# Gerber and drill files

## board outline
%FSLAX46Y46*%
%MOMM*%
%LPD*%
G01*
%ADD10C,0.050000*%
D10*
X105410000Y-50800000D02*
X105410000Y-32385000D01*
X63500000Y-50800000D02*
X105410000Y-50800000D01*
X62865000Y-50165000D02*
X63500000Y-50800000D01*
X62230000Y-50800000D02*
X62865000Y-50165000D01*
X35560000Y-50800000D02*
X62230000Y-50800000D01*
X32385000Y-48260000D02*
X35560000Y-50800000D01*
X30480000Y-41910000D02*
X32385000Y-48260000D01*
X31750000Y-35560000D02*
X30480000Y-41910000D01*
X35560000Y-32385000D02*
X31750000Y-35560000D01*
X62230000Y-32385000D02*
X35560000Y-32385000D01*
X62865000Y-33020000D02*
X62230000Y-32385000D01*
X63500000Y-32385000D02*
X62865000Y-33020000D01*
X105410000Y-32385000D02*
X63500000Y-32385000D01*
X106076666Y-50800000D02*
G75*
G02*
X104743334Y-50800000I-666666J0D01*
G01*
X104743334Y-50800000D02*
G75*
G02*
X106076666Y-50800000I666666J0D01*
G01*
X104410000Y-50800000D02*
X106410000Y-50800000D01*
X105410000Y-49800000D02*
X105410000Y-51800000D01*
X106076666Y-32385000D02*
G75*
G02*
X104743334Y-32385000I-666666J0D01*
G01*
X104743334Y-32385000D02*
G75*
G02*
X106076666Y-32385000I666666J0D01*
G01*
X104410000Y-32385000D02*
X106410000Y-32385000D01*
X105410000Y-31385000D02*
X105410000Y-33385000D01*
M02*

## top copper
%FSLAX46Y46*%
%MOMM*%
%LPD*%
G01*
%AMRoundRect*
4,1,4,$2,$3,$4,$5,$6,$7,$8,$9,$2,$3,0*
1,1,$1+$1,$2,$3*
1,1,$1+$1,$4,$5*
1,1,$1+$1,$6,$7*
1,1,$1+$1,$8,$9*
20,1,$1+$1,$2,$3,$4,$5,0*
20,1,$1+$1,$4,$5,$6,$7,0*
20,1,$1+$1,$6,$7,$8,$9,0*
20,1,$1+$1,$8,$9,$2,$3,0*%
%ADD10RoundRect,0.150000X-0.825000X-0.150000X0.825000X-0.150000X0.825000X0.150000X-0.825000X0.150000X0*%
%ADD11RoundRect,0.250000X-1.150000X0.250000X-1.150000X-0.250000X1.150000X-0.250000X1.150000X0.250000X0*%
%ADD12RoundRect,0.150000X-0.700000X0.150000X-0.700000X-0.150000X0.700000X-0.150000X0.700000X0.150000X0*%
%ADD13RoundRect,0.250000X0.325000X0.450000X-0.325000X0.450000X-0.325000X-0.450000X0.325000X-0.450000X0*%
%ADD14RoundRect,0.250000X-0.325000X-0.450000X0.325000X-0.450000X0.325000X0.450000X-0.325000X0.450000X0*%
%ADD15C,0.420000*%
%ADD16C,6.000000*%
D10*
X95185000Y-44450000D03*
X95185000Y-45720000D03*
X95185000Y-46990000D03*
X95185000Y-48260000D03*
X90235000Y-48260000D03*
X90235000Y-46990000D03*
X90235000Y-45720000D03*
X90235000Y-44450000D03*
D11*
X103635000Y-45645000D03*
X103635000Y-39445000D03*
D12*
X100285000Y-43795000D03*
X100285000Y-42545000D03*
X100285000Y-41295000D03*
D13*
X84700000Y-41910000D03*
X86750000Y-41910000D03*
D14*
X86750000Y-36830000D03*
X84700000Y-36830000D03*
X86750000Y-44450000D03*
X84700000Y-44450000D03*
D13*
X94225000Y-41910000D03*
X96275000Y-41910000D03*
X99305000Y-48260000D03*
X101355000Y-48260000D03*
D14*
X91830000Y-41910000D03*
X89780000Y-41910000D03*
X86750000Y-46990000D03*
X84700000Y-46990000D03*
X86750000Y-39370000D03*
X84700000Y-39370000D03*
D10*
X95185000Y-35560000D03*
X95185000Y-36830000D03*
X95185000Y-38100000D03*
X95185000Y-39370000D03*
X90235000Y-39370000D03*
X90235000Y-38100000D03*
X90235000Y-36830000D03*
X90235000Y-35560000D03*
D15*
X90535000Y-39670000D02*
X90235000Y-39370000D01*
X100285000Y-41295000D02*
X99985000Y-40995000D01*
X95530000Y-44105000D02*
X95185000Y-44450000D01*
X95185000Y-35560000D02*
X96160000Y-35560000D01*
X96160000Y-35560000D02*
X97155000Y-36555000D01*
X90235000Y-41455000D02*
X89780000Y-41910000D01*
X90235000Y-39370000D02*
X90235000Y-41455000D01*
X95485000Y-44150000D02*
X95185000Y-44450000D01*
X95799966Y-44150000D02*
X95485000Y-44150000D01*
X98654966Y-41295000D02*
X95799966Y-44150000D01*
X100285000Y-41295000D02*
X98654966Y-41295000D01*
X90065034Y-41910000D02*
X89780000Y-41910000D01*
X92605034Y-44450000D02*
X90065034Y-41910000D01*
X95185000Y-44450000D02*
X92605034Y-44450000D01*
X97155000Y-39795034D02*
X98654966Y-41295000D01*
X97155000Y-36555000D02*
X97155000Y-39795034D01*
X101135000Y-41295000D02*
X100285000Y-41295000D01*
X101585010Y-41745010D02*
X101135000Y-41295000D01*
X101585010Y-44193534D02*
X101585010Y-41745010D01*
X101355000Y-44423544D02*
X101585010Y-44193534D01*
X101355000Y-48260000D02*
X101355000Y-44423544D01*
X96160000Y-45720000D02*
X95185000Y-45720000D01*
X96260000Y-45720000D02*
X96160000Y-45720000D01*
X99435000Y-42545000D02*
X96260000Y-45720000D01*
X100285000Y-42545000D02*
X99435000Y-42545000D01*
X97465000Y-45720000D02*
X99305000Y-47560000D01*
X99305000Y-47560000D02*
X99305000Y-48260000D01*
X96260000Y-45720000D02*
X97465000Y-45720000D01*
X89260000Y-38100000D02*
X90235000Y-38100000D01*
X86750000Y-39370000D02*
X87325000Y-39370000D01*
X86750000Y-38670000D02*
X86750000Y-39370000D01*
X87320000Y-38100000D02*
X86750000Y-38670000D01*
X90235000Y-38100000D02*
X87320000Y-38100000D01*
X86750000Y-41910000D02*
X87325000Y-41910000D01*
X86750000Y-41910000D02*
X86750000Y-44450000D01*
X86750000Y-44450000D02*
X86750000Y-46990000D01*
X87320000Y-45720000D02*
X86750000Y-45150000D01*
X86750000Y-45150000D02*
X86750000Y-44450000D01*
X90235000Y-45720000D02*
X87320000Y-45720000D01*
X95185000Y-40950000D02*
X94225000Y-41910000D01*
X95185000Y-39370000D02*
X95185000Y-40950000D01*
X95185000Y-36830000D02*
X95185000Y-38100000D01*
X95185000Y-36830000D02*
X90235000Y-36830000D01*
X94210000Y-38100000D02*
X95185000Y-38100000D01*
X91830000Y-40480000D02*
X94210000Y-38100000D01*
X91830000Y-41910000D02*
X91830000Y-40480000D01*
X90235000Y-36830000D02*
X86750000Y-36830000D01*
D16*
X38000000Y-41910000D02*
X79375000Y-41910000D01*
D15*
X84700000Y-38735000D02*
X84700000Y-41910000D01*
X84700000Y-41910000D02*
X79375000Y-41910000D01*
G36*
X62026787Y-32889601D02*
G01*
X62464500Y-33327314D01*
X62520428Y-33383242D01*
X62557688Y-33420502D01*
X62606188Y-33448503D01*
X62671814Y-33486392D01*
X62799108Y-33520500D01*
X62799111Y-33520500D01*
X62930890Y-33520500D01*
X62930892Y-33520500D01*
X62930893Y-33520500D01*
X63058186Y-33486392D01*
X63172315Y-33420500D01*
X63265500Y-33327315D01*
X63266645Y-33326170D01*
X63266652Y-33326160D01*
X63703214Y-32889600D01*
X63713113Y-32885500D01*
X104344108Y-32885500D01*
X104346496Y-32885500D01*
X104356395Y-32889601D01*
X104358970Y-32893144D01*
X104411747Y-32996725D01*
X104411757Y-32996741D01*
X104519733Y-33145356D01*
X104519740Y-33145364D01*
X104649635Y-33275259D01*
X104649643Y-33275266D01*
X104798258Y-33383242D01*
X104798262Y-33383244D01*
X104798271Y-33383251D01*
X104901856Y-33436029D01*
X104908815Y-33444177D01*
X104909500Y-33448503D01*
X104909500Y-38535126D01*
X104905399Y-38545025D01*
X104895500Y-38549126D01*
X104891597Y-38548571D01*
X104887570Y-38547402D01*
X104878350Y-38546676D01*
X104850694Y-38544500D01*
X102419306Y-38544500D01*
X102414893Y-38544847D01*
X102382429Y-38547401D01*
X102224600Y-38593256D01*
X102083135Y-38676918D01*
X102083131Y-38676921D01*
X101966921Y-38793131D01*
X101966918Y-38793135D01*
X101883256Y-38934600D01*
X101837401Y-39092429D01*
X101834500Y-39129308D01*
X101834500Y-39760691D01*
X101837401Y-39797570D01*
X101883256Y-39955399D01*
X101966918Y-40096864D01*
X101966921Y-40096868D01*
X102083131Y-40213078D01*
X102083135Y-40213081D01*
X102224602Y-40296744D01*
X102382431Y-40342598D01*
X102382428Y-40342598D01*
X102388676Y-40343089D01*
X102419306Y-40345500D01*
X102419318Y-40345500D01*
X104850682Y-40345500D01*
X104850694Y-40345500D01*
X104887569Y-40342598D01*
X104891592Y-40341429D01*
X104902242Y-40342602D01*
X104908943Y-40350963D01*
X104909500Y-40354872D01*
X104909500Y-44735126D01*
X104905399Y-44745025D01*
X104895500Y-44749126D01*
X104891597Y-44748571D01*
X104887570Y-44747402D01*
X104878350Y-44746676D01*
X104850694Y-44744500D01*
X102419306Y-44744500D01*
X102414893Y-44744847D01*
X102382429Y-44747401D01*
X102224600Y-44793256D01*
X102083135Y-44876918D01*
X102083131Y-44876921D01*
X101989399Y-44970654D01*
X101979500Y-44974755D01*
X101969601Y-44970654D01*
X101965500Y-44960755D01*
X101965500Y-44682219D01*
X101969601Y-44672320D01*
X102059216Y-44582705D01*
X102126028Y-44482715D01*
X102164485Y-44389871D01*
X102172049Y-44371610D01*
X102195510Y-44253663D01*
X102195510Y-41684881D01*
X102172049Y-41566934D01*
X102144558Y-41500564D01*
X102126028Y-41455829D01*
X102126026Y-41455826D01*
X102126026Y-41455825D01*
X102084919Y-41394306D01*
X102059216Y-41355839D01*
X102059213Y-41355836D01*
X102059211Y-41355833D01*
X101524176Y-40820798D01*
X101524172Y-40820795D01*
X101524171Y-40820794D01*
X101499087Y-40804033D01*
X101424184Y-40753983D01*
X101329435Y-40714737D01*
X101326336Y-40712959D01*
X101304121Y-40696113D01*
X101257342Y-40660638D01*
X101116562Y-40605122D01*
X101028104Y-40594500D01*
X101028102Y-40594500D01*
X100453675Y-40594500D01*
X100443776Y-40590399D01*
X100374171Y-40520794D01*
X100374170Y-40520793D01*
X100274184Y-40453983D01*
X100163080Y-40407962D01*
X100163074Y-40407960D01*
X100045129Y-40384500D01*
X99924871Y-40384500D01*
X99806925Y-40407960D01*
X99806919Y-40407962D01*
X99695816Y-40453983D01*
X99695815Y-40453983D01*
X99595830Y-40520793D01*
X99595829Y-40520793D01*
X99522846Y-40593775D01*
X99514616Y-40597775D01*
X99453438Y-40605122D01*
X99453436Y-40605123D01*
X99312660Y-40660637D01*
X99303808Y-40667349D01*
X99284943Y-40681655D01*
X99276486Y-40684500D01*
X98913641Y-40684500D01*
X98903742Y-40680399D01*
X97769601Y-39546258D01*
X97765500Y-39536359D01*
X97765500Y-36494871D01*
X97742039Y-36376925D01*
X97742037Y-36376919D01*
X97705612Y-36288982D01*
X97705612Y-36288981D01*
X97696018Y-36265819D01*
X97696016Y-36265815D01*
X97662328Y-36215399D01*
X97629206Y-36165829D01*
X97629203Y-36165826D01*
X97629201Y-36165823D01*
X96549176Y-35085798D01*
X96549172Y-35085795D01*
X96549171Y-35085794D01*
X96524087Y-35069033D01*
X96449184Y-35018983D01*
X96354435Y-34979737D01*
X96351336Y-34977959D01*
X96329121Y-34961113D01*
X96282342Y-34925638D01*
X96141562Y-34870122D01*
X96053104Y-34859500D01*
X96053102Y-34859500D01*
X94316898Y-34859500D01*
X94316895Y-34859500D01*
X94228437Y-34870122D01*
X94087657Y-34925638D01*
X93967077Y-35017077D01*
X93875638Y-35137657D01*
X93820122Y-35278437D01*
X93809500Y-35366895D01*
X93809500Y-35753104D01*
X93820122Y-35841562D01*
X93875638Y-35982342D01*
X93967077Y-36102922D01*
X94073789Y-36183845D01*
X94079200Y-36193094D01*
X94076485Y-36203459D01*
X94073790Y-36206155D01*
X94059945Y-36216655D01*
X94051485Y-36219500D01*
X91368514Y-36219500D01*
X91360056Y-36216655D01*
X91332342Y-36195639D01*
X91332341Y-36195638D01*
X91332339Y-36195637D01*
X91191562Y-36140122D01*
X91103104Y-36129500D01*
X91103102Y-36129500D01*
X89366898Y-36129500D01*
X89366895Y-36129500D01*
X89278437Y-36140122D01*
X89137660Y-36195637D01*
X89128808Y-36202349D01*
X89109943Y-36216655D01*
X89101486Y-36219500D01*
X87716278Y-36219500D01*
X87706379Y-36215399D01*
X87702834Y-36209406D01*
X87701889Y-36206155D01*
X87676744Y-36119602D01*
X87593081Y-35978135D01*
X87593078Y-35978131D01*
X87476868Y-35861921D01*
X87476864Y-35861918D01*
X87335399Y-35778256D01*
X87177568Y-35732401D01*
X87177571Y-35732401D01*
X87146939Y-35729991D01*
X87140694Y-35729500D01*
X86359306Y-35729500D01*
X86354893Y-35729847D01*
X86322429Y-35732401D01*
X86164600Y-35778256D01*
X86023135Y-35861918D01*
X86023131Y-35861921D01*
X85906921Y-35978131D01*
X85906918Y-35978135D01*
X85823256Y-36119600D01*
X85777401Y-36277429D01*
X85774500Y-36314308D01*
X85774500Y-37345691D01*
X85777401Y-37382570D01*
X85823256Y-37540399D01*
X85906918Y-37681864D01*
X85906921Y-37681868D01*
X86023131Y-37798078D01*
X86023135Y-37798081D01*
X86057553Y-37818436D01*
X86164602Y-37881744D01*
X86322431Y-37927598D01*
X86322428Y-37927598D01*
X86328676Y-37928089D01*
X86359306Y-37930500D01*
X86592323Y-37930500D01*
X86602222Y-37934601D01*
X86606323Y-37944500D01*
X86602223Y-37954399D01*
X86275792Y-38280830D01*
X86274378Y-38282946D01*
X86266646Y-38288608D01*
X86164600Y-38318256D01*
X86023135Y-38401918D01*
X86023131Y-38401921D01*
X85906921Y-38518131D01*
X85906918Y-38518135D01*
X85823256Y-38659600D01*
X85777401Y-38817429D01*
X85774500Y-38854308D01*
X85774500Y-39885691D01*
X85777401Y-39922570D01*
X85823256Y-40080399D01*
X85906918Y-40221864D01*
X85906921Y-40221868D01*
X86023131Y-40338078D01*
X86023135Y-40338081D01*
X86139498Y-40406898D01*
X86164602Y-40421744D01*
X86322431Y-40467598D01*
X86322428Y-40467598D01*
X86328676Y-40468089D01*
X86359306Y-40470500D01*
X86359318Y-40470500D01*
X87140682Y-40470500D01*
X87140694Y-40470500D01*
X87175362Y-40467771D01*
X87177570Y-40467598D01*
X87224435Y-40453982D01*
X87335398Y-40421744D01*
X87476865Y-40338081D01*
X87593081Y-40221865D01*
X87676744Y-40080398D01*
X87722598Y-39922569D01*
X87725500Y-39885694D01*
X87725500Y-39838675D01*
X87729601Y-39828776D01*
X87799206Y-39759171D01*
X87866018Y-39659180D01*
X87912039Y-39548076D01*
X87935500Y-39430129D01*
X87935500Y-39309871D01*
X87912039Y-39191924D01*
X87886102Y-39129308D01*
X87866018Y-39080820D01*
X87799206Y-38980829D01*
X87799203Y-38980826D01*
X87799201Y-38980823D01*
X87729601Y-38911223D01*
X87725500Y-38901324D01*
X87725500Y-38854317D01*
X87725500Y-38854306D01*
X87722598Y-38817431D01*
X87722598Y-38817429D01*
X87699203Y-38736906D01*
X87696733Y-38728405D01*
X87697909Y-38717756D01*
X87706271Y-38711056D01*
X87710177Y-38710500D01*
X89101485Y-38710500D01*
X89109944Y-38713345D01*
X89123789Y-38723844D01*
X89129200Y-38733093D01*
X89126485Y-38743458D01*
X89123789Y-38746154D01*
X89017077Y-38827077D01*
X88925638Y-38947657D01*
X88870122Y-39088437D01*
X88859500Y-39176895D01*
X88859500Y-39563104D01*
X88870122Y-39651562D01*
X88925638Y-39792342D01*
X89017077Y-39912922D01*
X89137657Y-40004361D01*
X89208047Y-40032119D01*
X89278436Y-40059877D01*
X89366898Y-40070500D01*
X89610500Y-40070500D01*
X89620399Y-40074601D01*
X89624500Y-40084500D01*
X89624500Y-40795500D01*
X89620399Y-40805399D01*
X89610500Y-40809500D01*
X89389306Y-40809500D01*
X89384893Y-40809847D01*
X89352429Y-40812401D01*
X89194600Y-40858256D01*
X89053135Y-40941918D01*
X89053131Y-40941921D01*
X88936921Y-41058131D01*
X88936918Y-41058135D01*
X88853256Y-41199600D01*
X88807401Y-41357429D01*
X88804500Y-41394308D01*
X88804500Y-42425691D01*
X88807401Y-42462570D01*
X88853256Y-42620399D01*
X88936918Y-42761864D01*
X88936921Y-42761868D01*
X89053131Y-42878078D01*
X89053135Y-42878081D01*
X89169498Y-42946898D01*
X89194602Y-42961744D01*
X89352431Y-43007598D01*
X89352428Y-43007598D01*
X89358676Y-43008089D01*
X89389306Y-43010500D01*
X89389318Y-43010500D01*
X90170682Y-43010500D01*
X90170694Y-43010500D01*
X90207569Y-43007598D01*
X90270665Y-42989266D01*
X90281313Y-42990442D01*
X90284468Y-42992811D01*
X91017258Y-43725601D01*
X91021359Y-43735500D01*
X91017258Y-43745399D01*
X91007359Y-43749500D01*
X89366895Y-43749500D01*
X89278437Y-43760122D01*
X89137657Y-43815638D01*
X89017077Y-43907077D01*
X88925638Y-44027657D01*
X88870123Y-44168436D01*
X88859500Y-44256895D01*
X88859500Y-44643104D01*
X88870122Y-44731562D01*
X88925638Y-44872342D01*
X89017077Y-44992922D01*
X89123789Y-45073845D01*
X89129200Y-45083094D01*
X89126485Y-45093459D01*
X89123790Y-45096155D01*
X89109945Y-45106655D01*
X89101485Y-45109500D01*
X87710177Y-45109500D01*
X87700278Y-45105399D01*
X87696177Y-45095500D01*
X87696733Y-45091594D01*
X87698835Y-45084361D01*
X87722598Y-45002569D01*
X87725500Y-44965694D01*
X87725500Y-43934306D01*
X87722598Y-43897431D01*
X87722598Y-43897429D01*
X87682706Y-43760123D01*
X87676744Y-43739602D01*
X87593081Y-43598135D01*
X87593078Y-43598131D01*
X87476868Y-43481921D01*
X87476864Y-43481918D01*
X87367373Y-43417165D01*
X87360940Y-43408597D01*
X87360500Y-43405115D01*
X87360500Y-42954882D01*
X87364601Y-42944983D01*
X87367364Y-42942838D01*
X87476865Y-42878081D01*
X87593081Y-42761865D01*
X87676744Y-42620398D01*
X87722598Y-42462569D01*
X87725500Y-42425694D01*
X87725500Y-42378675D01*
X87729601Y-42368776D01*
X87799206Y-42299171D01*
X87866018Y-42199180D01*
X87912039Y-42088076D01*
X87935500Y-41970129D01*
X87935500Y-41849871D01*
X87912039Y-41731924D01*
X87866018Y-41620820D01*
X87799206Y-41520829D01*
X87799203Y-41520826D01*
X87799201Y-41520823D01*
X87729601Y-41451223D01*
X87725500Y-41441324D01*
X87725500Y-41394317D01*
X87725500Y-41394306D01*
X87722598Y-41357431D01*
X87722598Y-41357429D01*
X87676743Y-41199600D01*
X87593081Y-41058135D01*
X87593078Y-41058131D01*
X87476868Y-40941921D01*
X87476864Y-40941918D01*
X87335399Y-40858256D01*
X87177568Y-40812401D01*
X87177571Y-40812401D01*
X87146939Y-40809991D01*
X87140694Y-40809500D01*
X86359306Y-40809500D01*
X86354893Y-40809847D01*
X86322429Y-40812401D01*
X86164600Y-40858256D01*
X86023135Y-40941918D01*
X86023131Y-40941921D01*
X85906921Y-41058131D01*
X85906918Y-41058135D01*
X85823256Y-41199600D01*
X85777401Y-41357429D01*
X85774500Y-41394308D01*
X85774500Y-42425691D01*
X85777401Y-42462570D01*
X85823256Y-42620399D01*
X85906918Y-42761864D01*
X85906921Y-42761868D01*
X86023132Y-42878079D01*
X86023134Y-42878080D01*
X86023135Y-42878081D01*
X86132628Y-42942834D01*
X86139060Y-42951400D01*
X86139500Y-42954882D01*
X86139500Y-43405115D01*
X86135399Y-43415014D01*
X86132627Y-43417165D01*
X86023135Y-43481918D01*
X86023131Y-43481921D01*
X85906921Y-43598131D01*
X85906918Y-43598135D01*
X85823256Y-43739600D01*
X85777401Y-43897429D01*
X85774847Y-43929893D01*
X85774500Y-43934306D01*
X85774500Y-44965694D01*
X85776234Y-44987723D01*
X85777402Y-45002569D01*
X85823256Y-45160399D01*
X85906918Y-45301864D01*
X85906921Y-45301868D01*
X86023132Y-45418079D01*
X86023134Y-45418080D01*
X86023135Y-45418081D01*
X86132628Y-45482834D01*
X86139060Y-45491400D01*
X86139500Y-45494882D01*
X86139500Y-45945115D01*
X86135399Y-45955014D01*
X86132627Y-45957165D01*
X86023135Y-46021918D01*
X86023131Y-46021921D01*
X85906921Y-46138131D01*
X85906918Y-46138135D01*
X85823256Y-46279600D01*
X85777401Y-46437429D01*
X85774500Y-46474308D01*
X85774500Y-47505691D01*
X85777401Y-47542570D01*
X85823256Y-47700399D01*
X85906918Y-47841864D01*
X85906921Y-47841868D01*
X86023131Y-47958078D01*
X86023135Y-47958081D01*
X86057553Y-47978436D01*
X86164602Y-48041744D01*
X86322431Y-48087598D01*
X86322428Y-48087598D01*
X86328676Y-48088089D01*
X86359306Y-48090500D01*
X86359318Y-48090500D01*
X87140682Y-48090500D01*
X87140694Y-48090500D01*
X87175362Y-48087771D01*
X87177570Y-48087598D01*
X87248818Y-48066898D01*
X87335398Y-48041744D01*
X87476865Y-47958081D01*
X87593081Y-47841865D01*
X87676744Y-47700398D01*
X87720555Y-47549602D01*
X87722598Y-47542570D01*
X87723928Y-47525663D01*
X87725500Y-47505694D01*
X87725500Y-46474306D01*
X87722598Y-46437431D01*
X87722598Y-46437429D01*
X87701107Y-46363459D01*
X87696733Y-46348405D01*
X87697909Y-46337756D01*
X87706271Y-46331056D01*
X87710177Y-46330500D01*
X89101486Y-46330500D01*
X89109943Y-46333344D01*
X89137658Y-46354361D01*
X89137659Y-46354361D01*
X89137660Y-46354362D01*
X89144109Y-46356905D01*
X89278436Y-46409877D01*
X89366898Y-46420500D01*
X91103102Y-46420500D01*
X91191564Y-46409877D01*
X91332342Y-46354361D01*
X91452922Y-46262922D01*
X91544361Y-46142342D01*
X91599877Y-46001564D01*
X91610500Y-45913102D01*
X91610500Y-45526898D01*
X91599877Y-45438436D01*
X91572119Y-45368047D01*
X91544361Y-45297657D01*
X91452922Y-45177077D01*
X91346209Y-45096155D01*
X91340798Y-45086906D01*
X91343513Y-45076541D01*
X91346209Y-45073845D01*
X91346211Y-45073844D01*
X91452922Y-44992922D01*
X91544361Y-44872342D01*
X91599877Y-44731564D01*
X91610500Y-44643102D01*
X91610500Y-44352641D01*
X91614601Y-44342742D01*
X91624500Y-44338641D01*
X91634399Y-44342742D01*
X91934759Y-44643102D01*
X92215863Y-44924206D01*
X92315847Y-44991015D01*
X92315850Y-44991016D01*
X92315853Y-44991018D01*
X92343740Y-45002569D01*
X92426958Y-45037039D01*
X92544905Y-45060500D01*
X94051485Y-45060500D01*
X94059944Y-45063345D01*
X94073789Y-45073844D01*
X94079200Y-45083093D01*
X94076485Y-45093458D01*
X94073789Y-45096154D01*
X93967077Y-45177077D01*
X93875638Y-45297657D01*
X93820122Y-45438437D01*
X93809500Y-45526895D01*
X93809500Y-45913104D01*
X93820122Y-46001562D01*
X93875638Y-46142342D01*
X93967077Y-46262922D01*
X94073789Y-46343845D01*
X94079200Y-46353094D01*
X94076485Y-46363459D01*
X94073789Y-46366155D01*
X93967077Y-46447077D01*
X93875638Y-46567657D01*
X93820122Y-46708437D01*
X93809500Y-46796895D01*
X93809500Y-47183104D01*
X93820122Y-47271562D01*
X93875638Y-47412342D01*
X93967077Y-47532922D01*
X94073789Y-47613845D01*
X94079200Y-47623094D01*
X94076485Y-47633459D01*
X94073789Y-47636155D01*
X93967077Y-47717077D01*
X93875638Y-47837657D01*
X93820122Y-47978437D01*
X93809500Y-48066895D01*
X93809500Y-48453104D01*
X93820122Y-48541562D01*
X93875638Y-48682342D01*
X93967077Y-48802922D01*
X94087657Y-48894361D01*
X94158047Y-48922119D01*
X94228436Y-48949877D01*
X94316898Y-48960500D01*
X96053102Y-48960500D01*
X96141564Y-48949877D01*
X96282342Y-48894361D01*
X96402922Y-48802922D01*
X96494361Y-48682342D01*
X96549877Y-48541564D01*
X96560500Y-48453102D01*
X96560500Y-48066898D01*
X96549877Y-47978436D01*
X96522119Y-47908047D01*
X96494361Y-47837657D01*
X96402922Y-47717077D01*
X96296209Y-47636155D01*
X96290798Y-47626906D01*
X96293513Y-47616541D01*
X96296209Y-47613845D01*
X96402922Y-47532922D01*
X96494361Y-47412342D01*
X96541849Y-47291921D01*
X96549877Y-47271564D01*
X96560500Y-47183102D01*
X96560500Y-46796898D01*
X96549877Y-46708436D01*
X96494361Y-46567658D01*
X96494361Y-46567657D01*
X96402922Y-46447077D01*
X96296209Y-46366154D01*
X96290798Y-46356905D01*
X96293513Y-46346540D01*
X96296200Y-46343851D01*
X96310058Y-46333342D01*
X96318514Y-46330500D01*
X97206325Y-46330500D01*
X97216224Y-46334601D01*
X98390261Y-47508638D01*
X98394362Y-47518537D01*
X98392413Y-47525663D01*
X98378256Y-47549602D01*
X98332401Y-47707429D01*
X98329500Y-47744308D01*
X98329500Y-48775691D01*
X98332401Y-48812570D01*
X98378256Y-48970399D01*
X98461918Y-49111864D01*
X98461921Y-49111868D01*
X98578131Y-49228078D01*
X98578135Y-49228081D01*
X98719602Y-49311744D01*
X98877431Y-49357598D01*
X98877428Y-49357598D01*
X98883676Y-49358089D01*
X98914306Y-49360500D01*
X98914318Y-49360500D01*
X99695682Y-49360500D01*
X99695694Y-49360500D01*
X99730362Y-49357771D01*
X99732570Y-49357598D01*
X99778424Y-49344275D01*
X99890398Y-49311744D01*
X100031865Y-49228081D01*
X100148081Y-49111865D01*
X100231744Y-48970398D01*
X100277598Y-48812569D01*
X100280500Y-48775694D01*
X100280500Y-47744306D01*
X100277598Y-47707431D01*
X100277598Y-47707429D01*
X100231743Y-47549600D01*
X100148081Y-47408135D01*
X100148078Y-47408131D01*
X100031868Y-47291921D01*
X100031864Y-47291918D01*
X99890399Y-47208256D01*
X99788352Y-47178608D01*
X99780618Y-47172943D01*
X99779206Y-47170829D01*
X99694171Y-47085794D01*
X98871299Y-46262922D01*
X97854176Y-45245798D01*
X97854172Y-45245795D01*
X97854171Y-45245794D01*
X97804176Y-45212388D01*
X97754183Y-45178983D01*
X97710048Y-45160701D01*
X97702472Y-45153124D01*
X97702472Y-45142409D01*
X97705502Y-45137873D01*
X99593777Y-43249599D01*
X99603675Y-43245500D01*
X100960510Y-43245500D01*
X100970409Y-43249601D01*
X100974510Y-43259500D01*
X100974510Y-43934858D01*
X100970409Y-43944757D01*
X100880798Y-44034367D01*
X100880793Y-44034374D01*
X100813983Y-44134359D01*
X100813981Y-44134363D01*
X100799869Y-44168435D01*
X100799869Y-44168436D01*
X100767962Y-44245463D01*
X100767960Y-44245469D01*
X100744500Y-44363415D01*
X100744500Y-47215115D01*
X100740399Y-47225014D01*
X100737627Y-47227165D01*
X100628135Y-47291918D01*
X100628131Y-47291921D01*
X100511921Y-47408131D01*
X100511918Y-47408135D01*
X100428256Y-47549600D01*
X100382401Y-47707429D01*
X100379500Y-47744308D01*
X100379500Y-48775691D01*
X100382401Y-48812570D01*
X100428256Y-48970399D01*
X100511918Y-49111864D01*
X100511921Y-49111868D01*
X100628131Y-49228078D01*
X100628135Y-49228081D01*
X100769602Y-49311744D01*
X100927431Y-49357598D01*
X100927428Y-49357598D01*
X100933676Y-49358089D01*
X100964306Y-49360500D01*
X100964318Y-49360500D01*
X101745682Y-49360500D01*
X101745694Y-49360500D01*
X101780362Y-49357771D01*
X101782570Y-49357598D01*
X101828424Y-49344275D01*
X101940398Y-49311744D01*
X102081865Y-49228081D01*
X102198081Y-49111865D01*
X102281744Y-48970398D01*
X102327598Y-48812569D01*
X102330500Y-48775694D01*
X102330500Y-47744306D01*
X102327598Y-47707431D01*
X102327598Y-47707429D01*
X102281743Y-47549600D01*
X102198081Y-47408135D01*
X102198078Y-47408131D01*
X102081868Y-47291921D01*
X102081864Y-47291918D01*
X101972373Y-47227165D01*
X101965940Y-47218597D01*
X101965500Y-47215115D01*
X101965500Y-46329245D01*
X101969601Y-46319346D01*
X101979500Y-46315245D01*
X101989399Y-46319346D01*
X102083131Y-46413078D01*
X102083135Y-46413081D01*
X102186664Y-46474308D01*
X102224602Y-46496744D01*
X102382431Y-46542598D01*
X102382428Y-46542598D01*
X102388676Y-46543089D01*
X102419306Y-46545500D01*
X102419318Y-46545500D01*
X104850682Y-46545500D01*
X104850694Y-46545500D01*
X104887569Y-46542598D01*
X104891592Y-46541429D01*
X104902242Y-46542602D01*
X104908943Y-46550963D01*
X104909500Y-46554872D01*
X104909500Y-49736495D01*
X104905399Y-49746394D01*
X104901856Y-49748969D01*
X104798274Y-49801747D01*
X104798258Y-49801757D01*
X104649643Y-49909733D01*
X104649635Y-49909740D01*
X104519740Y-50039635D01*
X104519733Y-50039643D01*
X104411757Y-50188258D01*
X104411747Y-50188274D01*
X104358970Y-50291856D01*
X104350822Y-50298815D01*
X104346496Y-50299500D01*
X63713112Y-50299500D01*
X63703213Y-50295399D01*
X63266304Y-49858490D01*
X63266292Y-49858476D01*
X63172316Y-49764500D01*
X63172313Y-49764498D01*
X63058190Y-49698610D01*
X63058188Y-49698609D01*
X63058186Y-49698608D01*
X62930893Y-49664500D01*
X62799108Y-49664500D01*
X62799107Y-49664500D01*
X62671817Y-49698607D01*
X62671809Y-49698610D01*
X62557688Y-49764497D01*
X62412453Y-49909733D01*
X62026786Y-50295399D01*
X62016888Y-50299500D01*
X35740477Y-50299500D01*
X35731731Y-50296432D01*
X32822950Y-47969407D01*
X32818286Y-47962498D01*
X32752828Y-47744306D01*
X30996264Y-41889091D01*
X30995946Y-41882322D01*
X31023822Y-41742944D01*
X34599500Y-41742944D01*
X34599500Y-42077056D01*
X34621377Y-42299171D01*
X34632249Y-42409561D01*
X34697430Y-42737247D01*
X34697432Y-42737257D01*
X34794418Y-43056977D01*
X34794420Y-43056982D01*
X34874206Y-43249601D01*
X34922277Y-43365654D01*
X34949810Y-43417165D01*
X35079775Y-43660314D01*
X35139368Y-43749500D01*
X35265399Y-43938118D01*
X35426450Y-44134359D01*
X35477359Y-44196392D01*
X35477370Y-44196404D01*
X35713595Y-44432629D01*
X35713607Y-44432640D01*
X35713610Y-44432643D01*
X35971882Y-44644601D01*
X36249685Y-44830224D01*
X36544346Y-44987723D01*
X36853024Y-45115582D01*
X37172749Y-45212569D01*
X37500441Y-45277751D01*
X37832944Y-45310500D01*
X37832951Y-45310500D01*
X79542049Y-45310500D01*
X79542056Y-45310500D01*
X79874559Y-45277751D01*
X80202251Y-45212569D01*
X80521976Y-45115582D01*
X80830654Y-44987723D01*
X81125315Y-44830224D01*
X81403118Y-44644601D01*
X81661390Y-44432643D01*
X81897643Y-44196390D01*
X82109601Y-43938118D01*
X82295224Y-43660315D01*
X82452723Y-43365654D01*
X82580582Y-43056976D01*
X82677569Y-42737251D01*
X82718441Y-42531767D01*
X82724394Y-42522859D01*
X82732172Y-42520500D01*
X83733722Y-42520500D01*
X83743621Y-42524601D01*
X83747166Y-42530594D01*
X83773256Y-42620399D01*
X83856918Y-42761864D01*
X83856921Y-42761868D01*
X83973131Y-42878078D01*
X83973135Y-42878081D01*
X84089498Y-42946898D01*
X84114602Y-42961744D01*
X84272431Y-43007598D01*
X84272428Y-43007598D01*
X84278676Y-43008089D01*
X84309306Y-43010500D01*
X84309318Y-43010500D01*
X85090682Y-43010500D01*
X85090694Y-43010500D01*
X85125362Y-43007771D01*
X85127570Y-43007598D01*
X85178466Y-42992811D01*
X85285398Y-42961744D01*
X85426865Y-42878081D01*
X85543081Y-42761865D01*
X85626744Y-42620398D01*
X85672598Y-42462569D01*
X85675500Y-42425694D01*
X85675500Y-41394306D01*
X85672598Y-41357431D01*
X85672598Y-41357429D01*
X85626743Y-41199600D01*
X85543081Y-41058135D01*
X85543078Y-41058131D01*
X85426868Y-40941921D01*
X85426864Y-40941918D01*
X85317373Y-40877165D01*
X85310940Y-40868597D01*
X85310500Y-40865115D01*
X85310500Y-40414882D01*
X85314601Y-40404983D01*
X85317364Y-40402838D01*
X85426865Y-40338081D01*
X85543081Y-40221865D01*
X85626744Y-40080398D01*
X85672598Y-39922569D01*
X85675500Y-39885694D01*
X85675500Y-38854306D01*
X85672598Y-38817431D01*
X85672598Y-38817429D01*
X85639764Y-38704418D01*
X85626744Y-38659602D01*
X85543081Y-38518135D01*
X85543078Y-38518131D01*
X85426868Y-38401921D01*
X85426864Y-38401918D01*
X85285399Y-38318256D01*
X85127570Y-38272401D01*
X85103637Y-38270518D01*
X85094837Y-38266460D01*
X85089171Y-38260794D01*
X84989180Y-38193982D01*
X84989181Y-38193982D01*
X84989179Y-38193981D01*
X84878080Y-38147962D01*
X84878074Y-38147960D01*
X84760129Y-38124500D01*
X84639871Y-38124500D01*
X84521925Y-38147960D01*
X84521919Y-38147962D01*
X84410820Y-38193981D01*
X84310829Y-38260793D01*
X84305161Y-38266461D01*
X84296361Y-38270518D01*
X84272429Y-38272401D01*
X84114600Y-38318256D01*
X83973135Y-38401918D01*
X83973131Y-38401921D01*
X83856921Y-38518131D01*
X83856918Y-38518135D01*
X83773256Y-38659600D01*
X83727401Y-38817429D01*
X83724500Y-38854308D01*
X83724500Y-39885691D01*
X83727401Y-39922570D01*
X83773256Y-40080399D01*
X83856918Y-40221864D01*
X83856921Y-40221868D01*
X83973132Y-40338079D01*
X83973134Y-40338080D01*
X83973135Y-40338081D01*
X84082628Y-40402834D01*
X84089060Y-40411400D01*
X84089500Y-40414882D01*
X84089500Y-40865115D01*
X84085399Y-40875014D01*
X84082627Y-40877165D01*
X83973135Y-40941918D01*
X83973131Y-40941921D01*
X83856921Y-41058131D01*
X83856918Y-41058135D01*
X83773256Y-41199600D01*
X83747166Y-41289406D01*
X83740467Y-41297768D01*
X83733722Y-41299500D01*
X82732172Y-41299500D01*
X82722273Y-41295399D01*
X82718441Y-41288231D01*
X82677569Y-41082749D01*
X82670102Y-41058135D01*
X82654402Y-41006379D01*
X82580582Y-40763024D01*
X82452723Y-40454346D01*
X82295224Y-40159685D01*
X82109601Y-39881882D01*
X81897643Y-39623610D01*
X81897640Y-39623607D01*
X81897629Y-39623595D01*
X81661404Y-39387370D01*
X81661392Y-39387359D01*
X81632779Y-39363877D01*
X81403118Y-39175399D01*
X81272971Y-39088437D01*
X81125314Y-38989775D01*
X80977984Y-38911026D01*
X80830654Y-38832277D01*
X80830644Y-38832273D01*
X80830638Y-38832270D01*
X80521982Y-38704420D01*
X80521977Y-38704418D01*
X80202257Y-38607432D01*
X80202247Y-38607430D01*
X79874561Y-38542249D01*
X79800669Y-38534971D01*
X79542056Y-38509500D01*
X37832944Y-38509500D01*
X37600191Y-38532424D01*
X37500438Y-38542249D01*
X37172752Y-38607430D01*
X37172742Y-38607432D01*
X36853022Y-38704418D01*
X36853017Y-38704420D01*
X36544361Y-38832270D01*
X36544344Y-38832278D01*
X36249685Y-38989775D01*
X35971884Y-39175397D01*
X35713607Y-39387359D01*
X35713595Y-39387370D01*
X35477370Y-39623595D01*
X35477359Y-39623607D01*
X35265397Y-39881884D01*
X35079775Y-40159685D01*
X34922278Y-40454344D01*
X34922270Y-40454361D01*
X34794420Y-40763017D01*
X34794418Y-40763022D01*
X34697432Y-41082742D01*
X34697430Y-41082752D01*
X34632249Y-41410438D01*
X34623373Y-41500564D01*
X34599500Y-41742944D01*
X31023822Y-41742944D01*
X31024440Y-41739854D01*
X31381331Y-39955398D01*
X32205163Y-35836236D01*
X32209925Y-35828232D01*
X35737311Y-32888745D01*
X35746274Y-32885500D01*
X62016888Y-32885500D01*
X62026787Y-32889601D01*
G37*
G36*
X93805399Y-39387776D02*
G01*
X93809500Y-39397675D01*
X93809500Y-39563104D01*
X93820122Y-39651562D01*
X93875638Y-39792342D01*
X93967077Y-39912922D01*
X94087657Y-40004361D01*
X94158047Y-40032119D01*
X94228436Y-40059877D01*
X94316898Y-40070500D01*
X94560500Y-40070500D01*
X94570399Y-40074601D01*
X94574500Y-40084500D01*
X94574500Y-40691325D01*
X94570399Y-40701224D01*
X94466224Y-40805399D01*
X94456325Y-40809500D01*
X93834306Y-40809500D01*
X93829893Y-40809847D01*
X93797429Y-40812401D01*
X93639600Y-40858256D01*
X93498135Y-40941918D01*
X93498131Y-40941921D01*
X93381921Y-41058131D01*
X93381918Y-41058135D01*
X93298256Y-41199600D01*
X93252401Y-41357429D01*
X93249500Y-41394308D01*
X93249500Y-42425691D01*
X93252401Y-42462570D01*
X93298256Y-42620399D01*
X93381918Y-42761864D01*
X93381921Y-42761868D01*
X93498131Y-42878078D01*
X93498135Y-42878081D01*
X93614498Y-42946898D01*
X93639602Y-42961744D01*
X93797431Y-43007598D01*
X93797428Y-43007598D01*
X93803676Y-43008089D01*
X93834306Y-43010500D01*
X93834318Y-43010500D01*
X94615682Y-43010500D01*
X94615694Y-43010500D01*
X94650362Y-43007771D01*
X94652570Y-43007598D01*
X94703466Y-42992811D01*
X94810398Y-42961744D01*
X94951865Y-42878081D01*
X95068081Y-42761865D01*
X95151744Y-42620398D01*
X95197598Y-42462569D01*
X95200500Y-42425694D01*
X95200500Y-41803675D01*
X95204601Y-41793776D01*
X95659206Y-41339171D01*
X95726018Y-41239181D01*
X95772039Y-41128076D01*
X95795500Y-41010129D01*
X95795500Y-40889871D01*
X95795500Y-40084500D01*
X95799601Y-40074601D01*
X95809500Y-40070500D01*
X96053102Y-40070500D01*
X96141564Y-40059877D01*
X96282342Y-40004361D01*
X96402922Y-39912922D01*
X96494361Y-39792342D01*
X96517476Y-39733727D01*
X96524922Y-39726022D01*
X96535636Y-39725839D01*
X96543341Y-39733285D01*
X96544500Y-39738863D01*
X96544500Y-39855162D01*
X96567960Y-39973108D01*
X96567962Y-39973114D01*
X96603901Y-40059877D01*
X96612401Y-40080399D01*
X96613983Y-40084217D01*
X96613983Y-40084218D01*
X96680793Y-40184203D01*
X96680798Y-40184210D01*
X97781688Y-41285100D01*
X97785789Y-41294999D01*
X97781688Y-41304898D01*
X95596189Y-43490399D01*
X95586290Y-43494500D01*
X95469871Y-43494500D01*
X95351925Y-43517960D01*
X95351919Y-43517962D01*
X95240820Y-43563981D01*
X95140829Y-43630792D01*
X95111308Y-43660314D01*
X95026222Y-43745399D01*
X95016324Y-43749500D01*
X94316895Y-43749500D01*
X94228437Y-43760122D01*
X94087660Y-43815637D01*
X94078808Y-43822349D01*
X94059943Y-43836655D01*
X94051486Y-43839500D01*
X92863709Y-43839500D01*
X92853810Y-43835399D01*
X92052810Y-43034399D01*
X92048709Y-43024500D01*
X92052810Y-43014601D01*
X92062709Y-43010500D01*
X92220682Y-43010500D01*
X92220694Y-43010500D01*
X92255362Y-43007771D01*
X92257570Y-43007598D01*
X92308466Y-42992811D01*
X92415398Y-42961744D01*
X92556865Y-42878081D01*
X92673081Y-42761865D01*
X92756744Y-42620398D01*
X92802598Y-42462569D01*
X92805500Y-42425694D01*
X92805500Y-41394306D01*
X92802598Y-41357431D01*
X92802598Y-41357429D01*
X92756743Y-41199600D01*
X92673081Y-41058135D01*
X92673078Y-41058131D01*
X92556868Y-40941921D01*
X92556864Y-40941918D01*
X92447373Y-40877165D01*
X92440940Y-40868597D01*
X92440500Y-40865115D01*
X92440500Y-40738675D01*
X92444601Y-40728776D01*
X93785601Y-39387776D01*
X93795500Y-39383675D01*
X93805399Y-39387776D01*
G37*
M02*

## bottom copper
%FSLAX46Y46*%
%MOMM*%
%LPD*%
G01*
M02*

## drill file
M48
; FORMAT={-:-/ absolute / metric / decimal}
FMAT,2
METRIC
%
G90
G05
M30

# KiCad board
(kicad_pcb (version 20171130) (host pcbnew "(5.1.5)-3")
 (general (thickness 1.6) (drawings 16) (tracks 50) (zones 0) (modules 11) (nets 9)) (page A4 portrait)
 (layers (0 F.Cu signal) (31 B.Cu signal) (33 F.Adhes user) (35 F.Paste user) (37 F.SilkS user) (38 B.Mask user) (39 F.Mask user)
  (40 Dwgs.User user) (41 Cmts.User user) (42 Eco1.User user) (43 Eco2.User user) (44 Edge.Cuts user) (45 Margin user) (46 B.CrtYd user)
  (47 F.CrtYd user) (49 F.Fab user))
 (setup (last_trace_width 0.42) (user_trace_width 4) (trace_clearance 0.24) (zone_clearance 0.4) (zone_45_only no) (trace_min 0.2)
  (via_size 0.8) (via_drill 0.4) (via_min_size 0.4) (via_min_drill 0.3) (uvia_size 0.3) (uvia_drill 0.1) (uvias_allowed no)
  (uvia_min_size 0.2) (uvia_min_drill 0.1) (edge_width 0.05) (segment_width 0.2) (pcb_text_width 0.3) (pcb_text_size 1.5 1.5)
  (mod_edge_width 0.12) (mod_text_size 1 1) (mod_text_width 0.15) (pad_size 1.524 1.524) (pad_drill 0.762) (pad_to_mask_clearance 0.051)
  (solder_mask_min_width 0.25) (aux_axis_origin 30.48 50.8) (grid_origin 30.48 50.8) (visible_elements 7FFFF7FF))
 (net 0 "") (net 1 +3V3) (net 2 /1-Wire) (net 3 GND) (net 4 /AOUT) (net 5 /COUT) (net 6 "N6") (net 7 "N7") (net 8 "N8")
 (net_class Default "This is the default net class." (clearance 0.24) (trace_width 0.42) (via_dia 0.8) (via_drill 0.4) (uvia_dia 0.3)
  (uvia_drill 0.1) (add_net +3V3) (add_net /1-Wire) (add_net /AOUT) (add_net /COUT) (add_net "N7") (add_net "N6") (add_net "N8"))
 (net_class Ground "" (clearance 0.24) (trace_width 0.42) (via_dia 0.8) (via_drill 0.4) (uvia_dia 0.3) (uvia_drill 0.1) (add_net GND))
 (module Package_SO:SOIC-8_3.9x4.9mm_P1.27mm (layer F.Cu) (at 92.71 46.355)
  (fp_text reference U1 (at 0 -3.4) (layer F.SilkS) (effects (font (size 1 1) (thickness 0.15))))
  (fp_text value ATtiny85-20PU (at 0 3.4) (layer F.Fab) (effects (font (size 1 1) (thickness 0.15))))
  (pad 8 smd roundrect (at 2.475 -1.905) (size 1.95 0.6) (layers F.Cu F.Paste F.Mask) (roundrect_rratio 0.25) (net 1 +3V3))
  (pad 7 smd roundrect (at 2.475 -0.635) (size 1.95 0.6) (layers F.Cu F.Paste F.Mask) (roundrect_rratio 0.25) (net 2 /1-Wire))
  (pad 6 smd roundrect (at 2.475 0.635) (size 1.95 0.6) (layers F.Cu F.Paste F.Mask) (roundrect_rratio 0.25))
  (pad 5 smd roundrect (at 2.475 1.905) (size 1.95 0.6) (layers F.Cu F.Paste F.Mask) (roundrect_rratio 0.25))
  (pad 4 smd roundrect (at -2.475 1.905) (size 1.95 0.6) (layers F.Cu F.Paste F.Mask) (roundrect_rratio 0.25) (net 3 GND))
  (pad 3 smd roundrect (at -2.475 0.635) (size 1.95 0.6) (layers F.Cu F.Paste F.Mask) (roundrect_rratio 0.25) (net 3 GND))
  (pad 2 smd roundrect (at -2.475 -0.635) (size 1.95 0.6) (layers F.Cu F.Paste F.Mask) (roundrect_rratio 0.25) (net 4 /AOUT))
  (pad 1 smd roundrect (at -2.475 -1.905) (size 1.95 0.6) (layers F.Cu F.Paste F.Mask) (roundrect_rratio 0.25)))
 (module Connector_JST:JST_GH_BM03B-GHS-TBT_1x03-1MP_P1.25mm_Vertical (layer F.Cu) (at 102.235 42.545 270)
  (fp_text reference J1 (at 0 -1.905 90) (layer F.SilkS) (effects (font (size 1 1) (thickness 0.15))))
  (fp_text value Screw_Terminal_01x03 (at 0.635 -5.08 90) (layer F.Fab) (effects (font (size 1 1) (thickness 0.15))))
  (pad MP smd roundrect (at 3.1 -1.4 270) (size 1 2.8) (layers F.Cu F.Paste F.Mask) (roundrect_rratio 0.25))
  (pad MP smd roundrect (at -3.1 -1.4 270) (size 1 2.8) (layers F.Cu F.Paste F.Mask) (roundrect_rratio 0.25))
  (pad 3 smd roundrect (at 1.25 1.95 270) (size 0.6 1.7) (layers F.Cu F.Paste F.Mask) (roundrect_rratio 0.25) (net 3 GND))
  (pad 2 smd roundrect (at 0 1.95 270) (size 0.6 1.7) (layers F.Cu F.Paste F.Mask) (roundrect_rratio 0.25) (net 2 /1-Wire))
  (pad 1 smd roundrect (at -1.25 1.95 270) (size 0.6 1.7) (layers F.Cu F.Paste F.Mask) (roundrect_rratio 0.25) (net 1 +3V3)))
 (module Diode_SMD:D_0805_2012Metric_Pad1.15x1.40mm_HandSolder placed (layer F.Cu) (at 85.725 41.91 180)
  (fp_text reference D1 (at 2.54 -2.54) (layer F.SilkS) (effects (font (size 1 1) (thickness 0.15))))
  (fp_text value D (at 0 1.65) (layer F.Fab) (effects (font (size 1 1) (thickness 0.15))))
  (pad 2 smd roundrect (at 1.025 0 180) (size 1.15 1.4) (layers F.Cu F.Paste F.Mask) (roundrect_rratio 0.217391) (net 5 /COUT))
  (pad 1 smd roundrect (at -1.025 0 180) (size 1.15 1.4) (layers F.Cu F.Paste F.Mask) (roundrect_rratio 0.217391) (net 4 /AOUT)))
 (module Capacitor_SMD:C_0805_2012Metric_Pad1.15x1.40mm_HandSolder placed (layer F.Cu) (at 85.725 36.83)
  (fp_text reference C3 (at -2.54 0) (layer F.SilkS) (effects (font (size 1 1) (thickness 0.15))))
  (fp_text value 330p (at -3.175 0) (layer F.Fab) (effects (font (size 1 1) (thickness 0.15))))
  (pad 2 smd roundrect (at 1.025 0) (size 1.15 1.4) (layers F.Cu F.Paste F.Mask) (roundrect_rratio 0.217391) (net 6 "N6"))
  (pad 1 smd roundrect (at -1.025 0) (size 1.15 1.4) (layers F.Cu F.Paste F.Mask) (roundrect_rratio 0.217391) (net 3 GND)))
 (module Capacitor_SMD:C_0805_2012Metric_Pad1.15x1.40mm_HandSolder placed (layer F.Cu) (at 85.725 44.45)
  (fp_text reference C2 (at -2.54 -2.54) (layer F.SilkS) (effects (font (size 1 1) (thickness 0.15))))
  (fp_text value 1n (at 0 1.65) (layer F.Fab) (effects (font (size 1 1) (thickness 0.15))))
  (pad 2 smd roundrect (at 1.025 0) (size 1.15 1.4) (layers F.Cu F.Paste F.Mask) (roundrect_rratio 0.217391) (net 4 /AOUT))
  (pad 1 smd roundrect (at -1.025 0) (size 1.15 1.4) (layers F.Cu F.Paste F.Mask) (roundrect_rratio 0.217391) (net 3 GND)))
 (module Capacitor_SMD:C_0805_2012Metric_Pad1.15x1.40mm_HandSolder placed (layer F.Cu) (at 95.25 41.91 180)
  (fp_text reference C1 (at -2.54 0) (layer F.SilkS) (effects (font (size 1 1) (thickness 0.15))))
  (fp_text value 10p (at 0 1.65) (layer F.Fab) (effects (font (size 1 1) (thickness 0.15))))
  (pad 2 smd roundrect (at 1.025 0 180) (size 1.15 1.4) (layers F.Cu F.Paste F.Mask) (roundrect_rratio 0.217391) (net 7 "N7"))
  (pad 1 smd roundrect (at -1.025 0 180) (size 1.15 1.4) (layers F.Cu F.Paste F.Mask) (roundrect_rratio 0.217391) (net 3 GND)))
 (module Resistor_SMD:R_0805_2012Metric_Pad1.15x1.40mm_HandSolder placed (layer F.Cu) (at 100.33 48.26 180)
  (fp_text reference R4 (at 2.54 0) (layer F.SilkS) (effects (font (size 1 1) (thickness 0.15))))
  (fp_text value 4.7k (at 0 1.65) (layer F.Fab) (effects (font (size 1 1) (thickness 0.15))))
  (pad 2 smd roundrect (at 1.025 0 180) (size 1.15 1.4) (layers F.Cu F.Paste F.Mask) (roundrect_rratio 0.217391) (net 2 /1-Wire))
  (pad 1 smd roundrect (at -1.025 0 180) (size 1.15 1.4) (layers F.Cu F.Paste F.Mask) (roundrect_rratio 0.217391) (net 1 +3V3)))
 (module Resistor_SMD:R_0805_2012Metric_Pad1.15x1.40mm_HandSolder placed (layer F.Cu) (at 90.805 41.91)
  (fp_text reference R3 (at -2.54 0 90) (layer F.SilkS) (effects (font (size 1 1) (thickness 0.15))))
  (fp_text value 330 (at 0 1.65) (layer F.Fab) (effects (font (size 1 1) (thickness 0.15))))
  (pad 2 smd roundrect (at 1.025 0) (size 1.15 1.4) (layers F.Cu F.Paste F.Mask) (roundrect_rratio 0.217391) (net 6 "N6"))
  (pad 1 smd roundrect (at -1.025 0) (size 1.15 1.4) (layers F.Cu F.Paste F.Mask) (roundrect_rratio 0.217391) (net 1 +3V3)))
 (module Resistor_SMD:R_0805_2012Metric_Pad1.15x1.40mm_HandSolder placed (layer F.Cu) (at 85.725 46.99)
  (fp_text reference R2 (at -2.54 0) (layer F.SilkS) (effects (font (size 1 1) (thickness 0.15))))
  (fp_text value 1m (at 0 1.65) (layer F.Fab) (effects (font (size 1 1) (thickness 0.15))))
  (pad 2 smd roundrect (at 1.025 0) (size 1.15 1.4) (layers F.Cu F.Paste F.Mask) (roundrect_rratio 0.217391) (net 4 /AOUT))
  (pad 1 smd roundrect (at -1.025 0) (size 1.15 1.4) (layers F.Cu F.Paste F.Mask) (roundrect_rratio 0.217391) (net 3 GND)))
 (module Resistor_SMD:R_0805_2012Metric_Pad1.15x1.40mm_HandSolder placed (layer F.Cu) (at 85.725 39.37)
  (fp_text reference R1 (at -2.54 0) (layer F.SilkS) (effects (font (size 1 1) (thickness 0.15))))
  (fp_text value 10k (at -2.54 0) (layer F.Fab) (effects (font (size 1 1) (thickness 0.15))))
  (pad 2 smd roundrect (at 1.025 0) (size 1.15 1.4) (layers F.Cu F.Paste F.Mask) (roundrect_rratio 0.217391) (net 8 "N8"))
  (pad 1 smd roundrect (at -1.025 0) (size 1.15 1.4) (layers F.Cu F.Paste F.Mask) (roundrect_rratio 0.217391) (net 5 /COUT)))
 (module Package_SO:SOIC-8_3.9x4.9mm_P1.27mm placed (layer F.Cu) (at 92.71 37.465)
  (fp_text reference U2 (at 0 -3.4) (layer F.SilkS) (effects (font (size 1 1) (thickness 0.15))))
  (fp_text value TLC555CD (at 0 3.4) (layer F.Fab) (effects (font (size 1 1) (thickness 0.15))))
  (pad 8 smd roundrect (at 2.475 -1.905) (size 1.95 0.6) (layers F.Cu F.Paste F.Mask) (roundrect_rratio 0.25) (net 1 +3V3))
  (pad 7 smd roundrect (at 2.475 -0.635) (size 1.95 0.6) (layers F.Cu F.Paste F.Mask) (roundrect_rratio 0.25) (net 6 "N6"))
  (pad 6 smd roundrect (at 2.475 0.635) (size 1.95 0.6) (layers F.Cu F.Paste F.Mask) (roundrect_rratio 0.25) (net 6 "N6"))
  (pad 5 smd roundrect (at 2.475 1.905) (size 1.95 0.6) (layers F.Cu F.Paste F.Mask) (roundrect_rratio 0.25) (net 7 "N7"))
  (pad 4 smd roundrect (at -2.475 1.905) (size 1.95 0.6) (layers F.Cu F.Paste F.Mask) (roundrect_rratio 0.25) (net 1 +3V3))
  (pad 3 smd roundrect (at -2.475 0.635) (size 1.95 0.6) (layers F.Cu F.Paste F.Mask) (roundrect_rratio 0.25) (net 8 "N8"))
  (pad 2 smd roundrect (at -2.475 -0.635) (size 1.95 0.6) (layers F.Cu F.Paste F.Mask) (roundrect_rratio 0.25) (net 6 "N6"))
  (pad 1 smd roundrect (at -2.475 -1.905) (size 1.95 0.6) (layers F.Cu F.Paste F.Mask) (roundrect_rratio 0.25) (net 3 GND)))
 (gr_line (start 105.41 50.8) (end 105.41 32.385) (layer Edge.Cuts) (width 0.05))
 (gr_line (start 63.5 50.8) (end 105.41 50.8) (layer Edge.Cuts) (width 0.05))
 (gr_line (start 62.865 50.165) (end 63.5 50.8) (layer Edge.Cuts) (width 0.05))
 (gr_line (start 62.23 50.8) (end 62.865 50.165) (layer Edge.Cuts) (width 0.05))
 (gr_line (start 35.56 50.8) (end 62.23 50.8) (layer Edge.Cuts) (width 0.05))
 (gr_line (start 32.385 48.26) (end 35.56 50.8) (layer Edge.Cuts) (width 0.05))
 (gr_line (start 30.48 41.91) (end 32.385 48.26) (layer Edge.Cuts) (width 0.05))
 (gr_line (start 31.75 35.56) (end 30.48 41.91) (layer Edge.Cuts) (width 0.05))
 (gr_line (start 35.56 32.385) (end 31.75 35.56) (layer Edge.Cuts) (width 0.05))
 (gr_line (start 62.23 32.385) (end 35.56 32.385) (layer Edge.Cuts) (width 0.05))
 (gr_line (start 62.865 33.02) (end 62.23 32.385) (layer Edge.Cuts) (width 0.05))
 (gr_line (start 63.5 32.385) (end 62.865 33.02) (layer Edge.Cuts) (width 0.05))
 (gr_line (start 105.41 32.385) (end 63.5 32.385) (layer Edge.Cuts) (width 0.05))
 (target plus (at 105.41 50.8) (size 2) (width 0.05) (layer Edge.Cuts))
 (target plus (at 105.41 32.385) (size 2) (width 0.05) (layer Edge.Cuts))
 (segment (start 90.535 39.67) (end 90.235 39.37) (width 0.42) (layer F.Cu) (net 1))
 (segment (start 100.285 41.295) (end 99.985 40.995) (width 0.42) (layer F.Cu) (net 1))
 (segment (start 95.53 44.105) (end 95.185 44.45) (width 0.42) (layer F.Cu) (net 1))
 (segment (start 95.185 35.56) (end 96.16 35.56) (width 0.42) (layer F.Cu) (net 1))
 (segment (start 96.16 35.56) (end 97.155 36.555) (width 0.42) (layer F.Cu) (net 1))
 (segment (start 90.235 41.455) (end 89.78 41.91) (width 0.42) (layer F.Cu) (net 1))
 (segment (start 90.235 39.37) (end 90.235 41.455) (width 0.42) (layer F.Cu) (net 1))
 (segment (start 95.485 44.15) (end 95.185 44.45) (width 0.42) (layer F.Cu) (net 1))
 (segment (start 95.799966 44.15) (end 95.485 44.15) (width 0.42) (layer F.Cu) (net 1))
 (segment (start 98.654966 41.295) (end 95.799966 44.15) (width 0.42) (layer F.Cu) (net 1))
 (segment (start 100.285 41.295) (end 98.654966 41.295) (width 0.42) (layer F.Cu) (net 1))
 (segment (start 90.065034 41.91) (end 89.78 41.91) (width 0.42) (layer F.Cu) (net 1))
 (segment (start 92.605034 44.45) (end 90.065034 41.91) (width 0.42) (layer F.Cu) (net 1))
 (segment (start 95.185 44.45) (end 92.605034 44.45) (width 0.42) (layer F.Cu) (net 1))
 (segment (start 97.155 39.795034) (end 98.654966 41.295) (width 0.42) (layer F.Cu) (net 1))
 (segment (start 97.155 36.555) (end 97.155 39.795034) (width 0.42) (layer F.Cu) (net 1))
 (segment (start 101.135 41.295) (end 100.285 41.295) (width 0.42) (layer F.Cu) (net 1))
 (segment (start 101.58501 41.74501) (end 101.135 41.295) (width 0.42) (layer F.Cu) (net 1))
 (segment (start 101.58501 44.193534) (end 101.58501 41.74501) (width 0.42) (layer F.Cu) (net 1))
 (segment (start 101.355 44.423544) (end 101.58501 44.193534) (width 0.42) (layer F.Cu) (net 1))
 (segment (start 101.355 48.26) (end 101.355 44.423544) (width 0.42) (layer F.Cu) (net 1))
 (segment (start 96.16 45.72) (end 95.185 45.72) (width 0.42) (layer F.Cu) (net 2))
 (segment (start 96.26 45.72) (end 96.16 45.72) (width 0.42) (layer F.Cu) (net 2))
 (segment (start 99.435 42.545) (end 96.26 45.72) (width 0.42) (layer F.Cu) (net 2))
 (segment (start 100.285 42.545) (end 99.435 42.545) (width 0.42) (layer F.Cu) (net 2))
 (segment (start 97.465 45.72) (end 99.305 47.56) (width 0.42) (layer F.Cu) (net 2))
 (segment (start 99.305 47.56) (end 99.305 48.26) (width 0.42) (layer F.Cu) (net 2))
 (segment (start 96.26 45.72) (end 97.465 45.72) (width 0.42) (layer F.Cu) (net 2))
 (segment (start 89.26 38.1) (end 90.235 38.1) (width 0.42) (layer F.Cu) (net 8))
 (segment (start 86.75 39.37) (end 87.325 39.37) (width 0.42) (layer F.Cu) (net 8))
 (segment (start 86.75 38.67) (end 86.75 39.37) (width 0.42) (layer F.Cu) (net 8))
 (segment (start 87.32 38.1) (end 86.75 38.67) (width 0.42) (layer F.Cu) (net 8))
 (segment (start 90.235 38.1) (end 87.32 38.1) (width 0.42) (layer F.Cu) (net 8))
 (segment (start 86.75 41.91) (end 87.325 41.91) (width 0.42) (layer F.Cu) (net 4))
 (segment (start 86.75 41.91) (end 86.75 44.45) (width 0.42) (layer F.Cu) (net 4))
 (segment (start 86.75 44.45) (end 86.75 46.99) (width 0.42) (layer F.Cu) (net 4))
 (segment (start 87.32 45.72) (end 86.75 45.15) (width 0.42) (layer F.Cu) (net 4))
 (segment (start 86.75 45.15) (end 86.75 44.45) (width 0.42) (layer F.Cu) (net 4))
 (segment (start 90.235 45.72) (end 87.32 45.72) (width 0.42) (layer F.Cu) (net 4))
 (segment (start 95.185 40.95) (end 94.225 41.91) (width 0.42) (layer F.Cu) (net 7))
 (segment (start 95.185 39.37) (end 95.185 40.95) (width 0.42) (layer F.Cu) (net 7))
 (segment (start 95.185 36.83) (end 95.185 38.1) (width 0.42) (layer F.Cu) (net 6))
 (segment (start 95.185 36.83) (end 90.235 36.83) (width 0.42) (layer F.Cu) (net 6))
 (segment (start 94.21 38.1) (end 95.185 38.1) (width 0.42) (layer F.Cu) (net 6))
 (segment (start 91.83 40.48) (end 94.21 38.1) (width 0.42) (layer F.Cu) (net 6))
 (segment (start 91.83 41.91) (end 91.83 40.48) (width 0.42) (layer F.Cu) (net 6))
 (segment (start 90.235 36.83) (end 86.75 36.83) (width 0.42) (layer F.Cu) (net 6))
 (segment (start 38 41.91) (end 79.375 41.91) (width 6) (layer F.Cu) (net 5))
 (segment (start 84.7 38.735) (end 84.7 41.91) (width 0.42) (layer F.Cu) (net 5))
 (segment (start 84.7 41.91) (end 79.375 41.91) (width 0.42) (layer F.Cu) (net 5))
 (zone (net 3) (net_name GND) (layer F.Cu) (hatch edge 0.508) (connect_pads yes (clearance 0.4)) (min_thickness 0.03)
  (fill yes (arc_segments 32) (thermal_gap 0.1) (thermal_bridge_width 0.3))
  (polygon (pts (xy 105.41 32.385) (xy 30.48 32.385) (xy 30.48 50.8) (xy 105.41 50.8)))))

